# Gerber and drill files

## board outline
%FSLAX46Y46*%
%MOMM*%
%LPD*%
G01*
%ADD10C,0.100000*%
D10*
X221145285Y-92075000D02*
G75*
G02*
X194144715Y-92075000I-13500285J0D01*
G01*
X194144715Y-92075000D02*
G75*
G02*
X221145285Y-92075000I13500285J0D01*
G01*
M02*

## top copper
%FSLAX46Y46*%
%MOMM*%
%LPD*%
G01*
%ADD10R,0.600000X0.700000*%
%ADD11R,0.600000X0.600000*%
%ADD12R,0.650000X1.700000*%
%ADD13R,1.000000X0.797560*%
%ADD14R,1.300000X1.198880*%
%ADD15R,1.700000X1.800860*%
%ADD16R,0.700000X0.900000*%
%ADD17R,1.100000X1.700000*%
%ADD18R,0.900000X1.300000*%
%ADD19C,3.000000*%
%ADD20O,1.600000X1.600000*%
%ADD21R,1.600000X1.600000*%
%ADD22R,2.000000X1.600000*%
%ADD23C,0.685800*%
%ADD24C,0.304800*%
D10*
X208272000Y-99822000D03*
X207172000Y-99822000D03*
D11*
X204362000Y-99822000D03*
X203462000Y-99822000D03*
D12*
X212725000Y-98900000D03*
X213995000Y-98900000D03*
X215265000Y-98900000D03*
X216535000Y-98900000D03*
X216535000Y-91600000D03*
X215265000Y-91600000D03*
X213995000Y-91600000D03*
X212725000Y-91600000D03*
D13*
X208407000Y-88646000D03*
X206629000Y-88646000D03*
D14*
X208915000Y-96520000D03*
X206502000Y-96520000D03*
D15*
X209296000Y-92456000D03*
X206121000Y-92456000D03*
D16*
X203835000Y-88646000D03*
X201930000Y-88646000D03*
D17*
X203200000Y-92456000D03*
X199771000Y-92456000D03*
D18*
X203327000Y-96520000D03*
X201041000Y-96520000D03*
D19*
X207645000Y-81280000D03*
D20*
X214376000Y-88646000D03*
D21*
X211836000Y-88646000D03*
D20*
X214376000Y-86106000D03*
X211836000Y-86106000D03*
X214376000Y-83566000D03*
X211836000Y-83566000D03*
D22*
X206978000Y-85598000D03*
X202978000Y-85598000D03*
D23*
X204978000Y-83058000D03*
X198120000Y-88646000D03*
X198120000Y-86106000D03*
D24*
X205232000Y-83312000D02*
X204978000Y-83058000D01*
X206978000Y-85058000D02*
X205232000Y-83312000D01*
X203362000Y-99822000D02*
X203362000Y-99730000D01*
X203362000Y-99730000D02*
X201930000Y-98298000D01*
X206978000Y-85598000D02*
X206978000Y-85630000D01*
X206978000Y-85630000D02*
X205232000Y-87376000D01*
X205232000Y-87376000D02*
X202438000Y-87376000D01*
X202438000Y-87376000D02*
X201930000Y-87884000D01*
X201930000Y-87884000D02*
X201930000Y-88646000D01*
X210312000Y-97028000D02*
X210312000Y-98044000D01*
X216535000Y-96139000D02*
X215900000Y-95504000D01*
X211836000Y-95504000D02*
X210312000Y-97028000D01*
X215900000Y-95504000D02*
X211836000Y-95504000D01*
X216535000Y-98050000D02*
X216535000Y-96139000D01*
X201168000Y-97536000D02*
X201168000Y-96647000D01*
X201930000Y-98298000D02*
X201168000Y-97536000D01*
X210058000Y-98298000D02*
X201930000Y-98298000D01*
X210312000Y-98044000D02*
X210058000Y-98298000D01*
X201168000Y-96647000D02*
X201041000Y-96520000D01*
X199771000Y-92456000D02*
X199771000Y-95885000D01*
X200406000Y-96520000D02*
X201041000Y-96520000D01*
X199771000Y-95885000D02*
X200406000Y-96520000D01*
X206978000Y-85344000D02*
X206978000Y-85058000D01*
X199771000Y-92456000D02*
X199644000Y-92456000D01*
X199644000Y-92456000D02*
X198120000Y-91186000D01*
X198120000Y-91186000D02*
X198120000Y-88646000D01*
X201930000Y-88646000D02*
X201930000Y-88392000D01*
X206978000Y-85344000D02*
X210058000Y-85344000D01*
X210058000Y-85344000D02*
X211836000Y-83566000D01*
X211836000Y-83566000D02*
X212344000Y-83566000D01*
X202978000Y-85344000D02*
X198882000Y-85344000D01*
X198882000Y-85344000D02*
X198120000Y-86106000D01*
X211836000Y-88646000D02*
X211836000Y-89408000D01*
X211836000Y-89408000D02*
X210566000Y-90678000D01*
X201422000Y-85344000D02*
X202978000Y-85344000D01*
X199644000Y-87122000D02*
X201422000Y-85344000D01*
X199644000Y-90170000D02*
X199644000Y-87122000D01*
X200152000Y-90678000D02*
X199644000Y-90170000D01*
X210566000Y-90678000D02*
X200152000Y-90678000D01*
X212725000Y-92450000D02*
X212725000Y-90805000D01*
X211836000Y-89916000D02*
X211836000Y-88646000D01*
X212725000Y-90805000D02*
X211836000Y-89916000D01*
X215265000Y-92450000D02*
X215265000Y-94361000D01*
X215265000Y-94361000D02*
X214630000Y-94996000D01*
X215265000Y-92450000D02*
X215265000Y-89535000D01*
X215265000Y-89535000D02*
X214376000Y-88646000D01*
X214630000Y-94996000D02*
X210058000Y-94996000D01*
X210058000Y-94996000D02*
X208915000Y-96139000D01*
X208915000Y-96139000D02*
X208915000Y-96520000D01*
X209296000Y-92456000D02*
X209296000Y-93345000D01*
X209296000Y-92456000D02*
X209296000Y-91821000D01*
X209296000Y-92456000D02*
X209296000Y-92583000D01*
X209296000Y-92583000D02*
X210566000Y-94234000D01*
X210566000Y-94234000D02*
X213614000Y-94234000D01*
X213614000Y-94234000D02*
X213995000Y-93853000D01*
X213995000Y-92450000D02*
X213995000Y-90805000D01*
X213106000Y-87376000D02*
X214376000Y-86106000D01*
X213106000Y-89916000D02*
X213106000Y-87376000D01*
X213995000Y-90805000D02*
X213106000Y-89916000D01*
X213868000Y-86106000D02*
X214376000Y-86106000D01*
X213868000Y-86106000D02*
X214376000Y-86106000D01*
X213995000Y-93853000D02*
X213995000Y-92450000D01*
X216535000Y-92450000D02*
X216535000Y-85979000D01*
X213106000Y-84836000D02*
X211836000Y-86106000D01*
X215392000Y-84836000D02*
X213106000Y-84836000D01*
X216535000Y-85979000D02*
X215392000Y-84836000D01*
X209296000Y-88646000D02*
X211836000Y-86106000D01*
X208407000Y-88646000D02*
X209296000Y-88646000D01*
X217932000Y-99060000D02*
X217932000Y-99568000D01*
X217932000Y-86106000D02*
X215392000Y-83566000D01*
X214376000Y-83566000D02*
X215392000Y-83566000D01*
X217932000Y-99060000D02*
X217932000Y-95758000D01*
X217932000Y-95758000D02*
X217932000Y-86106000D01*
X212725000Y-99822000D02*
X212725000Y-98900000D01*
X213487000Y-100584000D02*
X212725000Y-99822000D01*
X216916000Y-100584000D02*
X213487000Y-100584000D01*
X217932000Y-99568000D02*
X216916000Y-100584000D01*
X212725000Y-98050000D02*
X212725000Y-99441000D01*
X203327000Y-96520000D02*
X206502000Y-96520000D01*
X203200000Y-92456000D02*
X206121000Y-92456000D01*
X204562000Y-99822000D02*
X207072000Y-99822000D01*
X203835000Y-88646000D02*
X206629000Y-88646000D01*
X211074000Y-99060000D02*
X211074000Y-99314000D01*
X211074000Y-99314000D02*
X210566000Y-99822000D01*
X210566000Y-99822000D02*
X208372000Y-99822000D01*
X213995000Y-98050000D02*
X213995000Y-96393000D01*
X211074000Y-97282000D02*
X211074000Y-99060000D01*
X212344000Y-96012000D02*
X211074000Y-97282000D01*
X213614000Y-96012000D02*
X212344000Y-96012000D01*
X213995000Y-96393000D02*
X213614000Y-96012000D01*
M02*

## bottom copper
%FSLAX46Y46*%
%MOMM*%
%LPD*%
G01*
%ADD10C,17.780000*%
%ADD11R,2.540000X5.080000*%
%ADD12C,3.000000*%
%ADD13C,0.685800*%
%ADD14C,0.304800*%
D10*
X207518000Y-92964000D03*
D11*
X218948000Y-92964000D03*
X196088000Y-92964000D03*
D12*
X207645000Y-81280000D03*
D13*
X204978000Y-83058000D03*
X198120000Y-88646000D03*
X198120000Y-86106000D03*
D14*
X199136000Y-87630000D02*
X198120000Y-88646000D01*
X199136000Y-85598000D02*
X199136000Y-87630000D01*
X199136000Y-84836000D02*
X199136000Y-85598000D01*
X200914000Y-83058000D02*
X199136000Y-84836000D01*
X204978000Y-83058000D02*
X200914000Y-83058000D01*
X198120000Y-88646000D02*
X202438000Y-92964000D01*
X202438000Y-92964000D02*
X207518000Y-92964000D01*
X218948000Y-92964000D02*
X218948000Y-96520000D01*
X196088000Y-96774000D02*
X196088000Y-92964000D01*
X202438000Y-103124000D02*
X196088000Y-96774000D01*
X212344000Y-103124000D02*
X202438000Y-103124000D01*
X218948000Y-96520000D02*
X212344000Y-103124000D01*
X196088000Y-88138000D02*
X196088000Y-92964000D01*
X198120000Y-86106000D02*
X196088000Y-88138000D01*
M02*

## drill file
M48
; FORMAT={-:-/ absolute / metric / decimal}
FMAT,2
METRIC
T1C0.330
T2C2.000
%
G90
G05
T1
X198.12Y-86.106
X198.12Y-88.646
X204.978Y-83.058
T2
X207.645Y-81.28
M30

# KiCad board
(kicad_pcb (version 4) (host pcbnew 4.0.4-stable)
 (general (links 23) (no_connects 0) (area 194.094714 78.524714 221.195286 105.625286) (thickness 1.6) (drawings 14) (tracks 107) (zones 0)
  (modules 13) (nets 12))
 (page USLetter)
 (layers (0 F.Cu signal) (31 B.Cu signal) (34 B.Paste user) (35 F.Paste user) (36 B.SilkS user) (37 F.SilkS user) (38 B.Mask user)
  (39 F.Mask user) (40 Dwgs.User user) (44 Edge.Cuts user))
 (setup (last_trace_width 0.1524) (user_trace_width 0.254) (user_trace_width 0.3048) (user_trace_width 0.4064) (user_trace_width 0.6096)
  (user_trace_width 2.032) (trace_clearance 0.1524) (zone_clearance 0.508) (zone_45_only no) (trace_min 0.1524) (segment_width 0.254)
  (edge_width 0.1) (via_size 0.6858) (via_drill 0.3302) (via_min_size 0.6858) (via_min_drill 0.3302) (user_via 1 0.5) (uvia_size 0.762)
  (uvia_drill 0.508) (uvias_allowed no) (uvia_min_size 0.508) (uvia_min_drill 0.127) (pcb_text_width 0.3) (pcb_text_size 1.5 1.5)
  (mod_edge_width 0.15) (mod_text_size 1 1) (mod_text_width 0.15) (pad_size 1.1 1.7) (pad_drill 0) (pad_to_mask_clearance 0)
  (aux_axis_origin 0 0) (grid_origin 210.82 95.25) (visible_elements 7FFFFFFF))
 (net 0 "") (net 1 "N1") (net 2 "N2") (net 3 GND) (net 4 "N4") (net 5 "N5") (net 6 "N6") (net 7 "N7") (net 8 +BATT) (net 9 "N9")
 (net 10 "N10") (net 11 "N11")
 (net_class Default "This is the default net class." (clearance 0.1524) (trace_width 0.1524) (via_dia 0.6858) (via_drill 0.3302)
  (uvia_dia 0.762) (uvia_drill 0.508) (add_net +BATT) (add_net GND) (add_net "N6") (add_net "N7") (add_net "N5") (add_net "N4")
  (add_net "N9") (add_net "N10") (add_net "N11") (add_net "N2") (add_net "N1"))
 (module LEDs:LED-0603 (layer F.Cu) (at 207.772 99.822)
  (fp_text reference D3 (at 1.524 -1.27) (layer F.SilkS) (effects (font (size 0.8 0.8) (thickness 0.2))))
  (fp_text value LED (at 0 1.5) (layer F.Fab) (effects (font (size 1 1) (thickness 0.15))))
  (pad 2 smd rect (at 0.5 0 180) (size 0.6 0.7) (layers F.Cu F.Paste F.Mask) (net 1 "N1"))
  (pad 1 smd rect (at -0.6 0 180) (size 0.6 0.7) (layers F.Cu F.Paste F.Mask) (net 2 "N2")))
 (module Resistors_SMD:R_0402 (layer F.Cu) (at 203.962 99.822 180)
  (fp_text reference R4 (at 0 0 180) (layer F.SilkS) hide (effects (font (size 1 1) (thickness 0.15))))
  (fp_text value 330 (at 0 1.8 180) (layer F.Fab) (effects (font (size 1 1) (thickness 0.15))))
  (pad 1 smd rect (at -0.4 0 180) (size 0.6 0.6) (layers F.Cu F.Paste F.Mask) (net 2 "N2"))
  (pad 2 smd rect (at 0.5 0 180) (size 0.6 0.6) (layers F.Cu F.Paste F.Mask) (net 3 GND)))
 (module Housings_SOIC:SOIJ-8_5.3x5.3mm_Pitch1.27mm (layer F.Cu) (at 214.63 95.25 90)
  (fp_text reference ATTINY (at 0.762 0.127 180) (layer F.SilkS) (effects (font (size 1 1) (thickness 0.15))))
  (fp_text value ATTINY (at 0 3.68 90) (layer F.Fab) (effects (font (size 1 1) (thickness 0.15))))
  (pad 1 smd rect (at -3.65 -1.905 90) (size 1.7 0.65) (layers F.Cu F.Paste F.Mask) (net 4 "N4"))
  (pad 2 smd rect (at -3.65 -0.635 90) (size 1.7 0.65) (layers F.Cu F.Paste F.Mask) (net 1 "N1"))
  (pad 3 smd rect (at -3.65 0.635 90) (size 1.7 0.65) (layers F.Cu F.Paste F.Mask))
  (pad 4 smd rect (at -3.65 1.905 90) (size 1.7 0.65) (layers F.Cu F.Paste F.Mask) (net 3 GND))
  (pad 5 smd rect (at 3.65 1.905 90) (size 1.7 0.65) (layers F.Cu F.Paste F.Mask) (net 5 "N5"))
  (pad 6 smd rect (at 3.65 0.635 90) (size 1.7 0.65) (layers F.Cu F.Paste F.Mask) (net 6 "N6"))
  (pad 7 smd rect (at 3.65 -0.635 90) (size 1.7 0.65) (layers F.Cu F.Paste F.Mask) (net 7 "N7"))
  (pad 8 smd rect (at 3.65 -1.905 90) (size 1.7 0.65) (layers F.Cu F.Paste F.Mask) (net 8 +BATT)))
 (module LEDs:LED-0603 (layer F.Cu) (at 207.518 88.646)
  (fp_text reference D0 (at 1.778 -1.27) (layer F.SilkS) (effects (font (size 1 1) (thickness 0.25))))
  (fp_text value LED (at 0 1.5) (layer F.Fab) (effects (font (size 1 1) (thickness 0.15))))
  (pad 2 smd rect (at 0.889 0 180) (size 1 0.79756) (layers F.Cu F.Paste F.Mask) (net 5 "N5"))
  (pad 1 smd rect (at -0.889 0 180) (size 1 0.79756) (layers F.Cu F.Paste F.Mask) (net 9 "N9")))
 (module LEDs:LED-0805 (layer F.Cu) (at 207.772 96.52)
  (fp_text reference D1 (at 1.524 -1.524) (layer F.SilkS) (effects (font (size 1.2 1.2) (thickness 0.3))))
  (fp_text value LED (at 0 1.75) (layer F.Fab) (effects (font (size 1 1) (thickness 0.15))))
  (pad 2 smd rect (at 1.143 0 180) (size 1.3 1.19888) (layers F.Cu F.Paste F.Mask) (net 6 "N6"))
  (pad 1 smd rect (at -1.27 0 180) (size 1.3 1.19888) (layers F.Cu F.Paste F.Mask) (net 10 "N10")))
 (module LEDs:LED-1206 (layer F.Cu) (at 207.772 92.456)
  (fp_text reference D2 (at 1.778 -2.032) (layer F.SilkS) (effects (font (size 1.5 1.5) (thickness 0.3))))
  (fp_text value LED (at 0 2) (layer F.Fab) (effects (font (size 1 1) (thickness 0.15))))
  (pad 2 smd rect (at 1.524 0 180) (size 1.7 1.80086) (layers F.Cu F.Paste F.Mask) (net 7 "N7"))
  (pad 1 smd rect (at -1.651 0 180) (size 1.7 1.80086) (layers F.Cu F.Paste F.Mask) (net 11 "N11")))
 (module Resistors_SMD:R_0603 (layer F.Cu) (at 202.946 88.646 180)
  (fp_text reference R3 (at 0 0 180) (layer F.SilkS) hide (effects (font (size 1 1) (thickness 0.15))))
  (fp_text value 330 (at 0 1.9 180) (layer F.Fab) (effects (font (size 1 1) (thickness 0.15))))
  (pad 1 smd rect (at -0.889 0 180) (size 0.7 0.9) (layers F.Cu F.Paste F.Mask) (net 9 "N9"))
  (pad 2 smd rect (at 1.016 0 180) (size 0.7 0.9) (layers F.Cu F.Paste F.Mask) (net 3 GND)))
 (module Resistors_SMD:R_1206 (layer F.Cu) (at 201.422 92.456 180)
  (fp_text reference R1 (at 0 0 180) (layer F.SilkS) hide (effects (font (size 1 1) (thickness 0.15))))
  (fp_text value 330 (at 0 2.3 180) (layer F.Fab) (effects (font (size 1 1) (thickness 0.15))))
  (pad 1 smd rect (at -1.778 0 180) (size 1.1 1.7) (layers F.Cu F.Paste F.Mask) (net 11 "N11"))
  (pad 2 smd rect (at 1.651 0 180) (size 1.1 1.7) (layers F.Cu F.Paste F.Mask) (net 3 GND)))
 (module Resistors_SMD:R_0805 (layer F.Cu) (at 202.184 96.52 180)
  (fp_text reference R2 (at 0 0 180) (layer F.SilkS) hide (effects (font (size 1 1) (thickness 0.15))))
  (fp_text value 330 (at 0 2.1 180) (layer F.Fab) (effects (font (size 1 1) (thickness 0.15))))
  (pad 1 smd rect (at -1.143 0 180) (size 0.9 1.3) (layers F.Cu F.Paste F.Mask) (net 10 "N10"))
  (pad 2 smd rect (at 1.143 0 180) (size 0.9 1.3) (layers F.Cu F.Paste F.Mask) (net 3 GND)))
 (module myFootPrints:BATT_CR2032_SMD (layer B.Cu) (at 207.518 92.964 180)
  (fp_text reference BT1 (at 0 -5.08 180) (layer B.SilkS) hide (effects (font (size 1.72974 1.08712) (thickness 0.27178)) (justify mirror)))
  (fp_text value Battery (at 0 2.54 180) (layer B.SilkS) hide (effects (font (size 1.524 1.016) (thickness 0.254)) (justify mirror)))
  (pad 2 smd circle (at 0 0 180) (size 17.78 17.78) (layers B.Cu B.Paste B.Mask) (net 3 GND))
  (pad 1 smd rect (at -11.43 0 180) (size 2.54 5.08) (layers B.Cu B.Paste B.Mask) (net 8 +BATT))
  (pad 1 smd rect (at 11.43 0 180) (size 2.54 5.08) (layers B.Cu B.Paste B.Mask) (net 8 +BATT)))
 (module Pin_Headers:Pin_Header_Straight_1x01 (layer F.Cu) (at 207.645 81.28)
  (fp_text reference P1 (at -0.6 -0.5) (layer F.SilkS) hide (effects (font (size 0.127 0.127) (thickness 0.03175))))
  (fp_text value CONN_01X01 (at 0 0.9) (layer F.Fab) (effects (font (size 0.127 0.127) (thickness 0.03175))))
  (pad "" thru_hole circle (at 0 0) (size 3 3) (drill 2) (layers *.Cu *.Mask)))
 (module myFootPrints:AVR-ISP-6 (layer F.Cu) (at 214.376 88.646 180)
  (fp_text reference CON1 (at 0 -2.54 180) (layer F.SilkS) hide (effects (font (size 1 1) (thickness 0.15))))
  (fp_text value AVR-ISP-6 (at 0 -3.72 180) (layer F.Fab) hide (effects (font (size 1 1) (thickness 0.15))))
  (pad 1 smd oval (at 0 0 180) (size 1.6 1.6) (layers F.Cu F.Paste F.Mask) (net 6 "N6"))
  (pad 2 smd rect (at 2.54 0 180) (size 1.6 1.6) (layers F.Cu F.Paste F.Mask) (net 8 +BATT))
  (pad 3 smd oval (at 0 2.54 180) (size 1.6 1.6) (layers F.Cu F.Paste F.Mask) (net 7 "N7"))
  (pad 4 smd oval (at 2.54 2.54 180) (size 1.6 1.6) (layers F.Cu F.Paste F.Mask) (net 5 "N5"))
  (pad 5 smd oval (at 0 5.08 180) (size 1.6 1.6) (layers F.Cu F.Paste F.Mask) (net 4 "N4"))
  (pad 6 smd oval (at 2.54 5.08 180) (size 1.6 1.6) (layers F.Cu F.Paste F.Mask) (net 3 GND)))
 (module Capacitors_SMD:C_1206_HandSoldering (layer F.Cu) (at 204.978 85.598 180)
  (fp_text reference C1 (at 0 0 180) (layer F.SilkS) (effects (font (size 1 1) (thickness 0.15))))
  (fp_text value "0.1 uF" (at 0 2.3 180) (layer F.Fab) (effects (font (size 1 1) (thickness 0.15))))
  (pad 1 smd rect (at -2 0 180) (size 2 1.6) (layers F.Cu F.Paste F.Mask) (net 3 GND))
  (pad 2 smd rect (at 2 0 180) (size 2 1.6) (layers F.Cu F.Paste F.Mask) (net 8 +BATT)))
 (gr_circle (center 207.645 92.075) (end 197.485 83.185) (layer Edge.Cuts) (width 0.1))
 (segment (start 205.232 83.312) (end 204.978 83.058) (width 0.3048) (layer F.Cu) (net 3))
 (segment (start 206.978 85.058) (end 205.232 83.312) (width 0.3048) (layer F.Cu) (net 3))
 (segment (start 199.136 87.63) (end 198.12 88.646) (width 0.3048) (layer B.Cu) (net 3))
 (segment (start 199.136 85.598) (end 199.136 87.63) (width 0.3048) (layer B.Cu) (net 3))
 (segment (start 199.136 84.836) (end 199.136 85.598) (width 0.3048) (layer B.Cu) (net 3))
 (segment (start 200.914 83.058) (end 199.136 84.836) (width 0.3048) (layer B.Cu) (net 3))
 (segment (start 204.978 83.058) (end 200.914 83.058) (width 0.3048) (layer B.Cu) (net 3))
 (via (at 204.978 83.058) (size 0.6858) (drill 0.3302) (layers F.Cu B.Cu) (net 3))
 (segment (start 203.362 99.822) (end 203.362 99.73) (width 0.3048) (layer F.Cu) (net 3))
 (segment (start 203.362 99.73) (end 201.93 98.298) (width 0.3048) (layer F.Cu) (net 3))
 (segment (start 206.978 85.598) (end 206.978 85.63) (width 0.3048) (layer F.Cu) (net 3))
 (segment (start 206.978 85.63) (end 205.232 87.376) (width 0.3048) (layer F.Cu) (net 3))
 (segment (start 205.232 87.376) (end 202.438 87.376) (width 0.3048) (layer F.Cu) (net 3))
 (segment (start 202.438 87.376) (end 201.93 87.884) (width 0.3048) (layer F.Cu) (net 3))
 (segment (start 201.93 87.884) (end 201.93 88.646) (width 0.3048) (layer F.Cu) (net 3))
 (segment (start 210.312 97.028) (end 210.312 98.044) (width 0.3048) (layer F.Cu) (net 3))
 (segment (start 216.535 96.139) (end 215.9 95.504) (width 0.3048) (layer F.Cu) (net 3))
 (segment (start 211.836 95.504) (end 210.312 97.028) (width 0.3048) (layer F.Cu) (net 3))
 (segment (start 215.9 95.504) (end 211.836 95.504) (width 0.3048) (layer F.Cu) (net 3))
 (segment (start 216.535 98.05) (end 216.535 96.139) (width 0.3048) (layer F.Cu) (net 3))
 (segment (start 201.168 97.536) (end 201.168 96.647) (width 0.3048) (layer F.Cu) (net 3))
 (segment (start 201.93 98.298) (end 201.168 97.536) (width 0.3048) (layer F.Cu) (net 3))
 (segment (start 210.058 98.298) (end 201.93 98.298) (width 0.3048) (layer F.Cu) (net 3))
 (segment (start 210.312 98.044) (end 210.058 98.298) (width 0.3048) (layer F.Cu) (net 3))
 (segment (start 201.168 96.647) (end 201.041 96.52) (width 0.3048) (layer F.Cu) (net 3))
 (segment (start 199.771 92.456) (end 199.771 95.885) (width 0.3048) (layer F.Cu) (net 3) (status 10))
 (segment (start 200.406 96.52) (end 201.041 96.52) (width 0.3048) (layer F.Cu) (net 3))
 (segment (start 199.771 95.885) (end 200.406 96.52) (width 0.3048) (layer F.Cu) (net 3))
 (segment (start 206.978 85.344) (end 206.978 85.058) (width 0.3048) (layer F.Cu) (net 3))
 (segment (start 199.771 92.456) (end 199.644 92.456) (width 0.3048) (layer F.Cu) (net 3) (status 30))
 (segment (start 198.12 88.646) (end 202.438 92.964) (width 0.3048) (layer B.Cu) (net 3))
 (via (at 198.12 88.646) (size 0.6858) (drill 0.3302) (layers F.Cu B.Cu) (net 3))
 (segment (start 199.644 92.456) (end 198.12 91.186) (width 0.3048) (layer F.Cu) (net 3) (status 10))
 (segment (start 198.12 91.186) (end 198.12 88.646) (width 0.3048) (layer F.Cu) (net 3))
 (segment (start 202.438 92.964) (end 207.518 92.964) (width 0.3048) (layer B.Cu) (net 3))
 (segment (start 201.93 88.646) (end 201.93 88.392) (width 0.3048) (layer F.Cu) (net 3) (status 30))
 (segment (start 206.978 85.344) (end 210.058 85.344) (width 0.3048) (layer F.Cu) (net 3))
 (segment (start 210.058 85.344) (end 211.836 83.566) (width 0.3048) (layer F.Cu) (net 3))
 (segment (start 211.836 83.566) (end 212.344 83.566) (width 0.3048) (layer F.Cu) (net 3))
 (segment (start 218.948 92.964) (end 218.948 96.52) (width 0.3048) (layer B.Cu) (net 8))
 (segment (start 196.088 96.774) (end 196.088 92.964) (width 0.3048) (layer B.Cu) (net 8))
 (segment (start 202.438 103.124) (end 196.088 96.774) (width 0.3048) (layer B.Cu) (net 8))
 (segment (start 212.344 103.124) (end 202.438 103.124) (width 0.3048) (layer B.Cu) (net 8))
 (segment (start 218.948 96.52) (end 212.344 103.124) (width 0.3048) (layer B.Cu) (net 8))
 (segment (start 202.978 85.344) (end 198.882 85.344) (width 0.3048) (layer F.Cu) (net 8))
 (segment (start 196.088 88.138) (end 196.088 92.964) (width 0.3048) (layer B.Cu) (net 8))
 (segment (start 198.12 86.106) (end 196.088 88.138) (width 0.3048) (layer B.Cu) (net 8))
 (via (at 198.12 86.106) (size 0.6858) (drill 0.3302) (layers F.Cu B.Cu) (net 8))
 (segment (start 198.882 85.344) (end 198.12 86.106) (width 0.3048) (layer F.Cu) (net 8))
 (segment (start 211.836 88.646) (end 211.836 89.408) (width 0.3048) (layer F.Cu) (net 8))
 (segment (start 211.836 89.408) (end 210.566 90.678) (width 0.3048) (layer F.Cu) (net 8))
 (segment (start 201.422 85.344) (end 202.978 85.344) (width 0.3048) (layer F.Cu) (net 8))
 (segment (start 199.644 87.122) (end 201.422 85.344) (width 0.3048) (layer F.Cu) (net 8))
 (segment (start 199.644 90.17) (end 199.644 87.122) (width 0.3048) (layer F.Cu) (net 8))
 (segment (start 200.152 90.678) (end 199.644 90.17) (width 0.3048) (layer F.Cu) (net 8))
 (segment (start 210.566 90.678) (end 200.152 90.678) (width 0.3048) (layer F.Cu) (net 8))
 (segment (start 212.725 92.45) (end 212.725 90.805) (width 0.3048) (layer F.Cu) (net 8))
 (segment (start 211.836 89.916) (end 211.836 88.646) (width 0.3048) (layer F.Cu) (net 8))
 (segment (start 212.725 90.805) (end 211.836 89.916) (width 0.3048) (layer F.Cu) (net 8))
 (segment (start 215.265 92.45) (end 215.265 94.361) (width 0.3048) (layer F.Cu) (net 6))
 (segment (start 215.265 94.361) (end 214.63 94.996) (width 0.3048) (layer F.Cu) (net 6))
 (segment (start 215.265 92.45) (end 215.265 89.535) (width 0.3048) (layer F.Cu) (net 6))
 (segment (start 215.265 89.535) (end 214.376 88.646) (width 0.3048) (layer F.Cu) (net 6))
 (segment (start 214.63 94.996) (end 210.058 94.996) (width 0.3048) (layer F.Cu) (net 6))
 (segment (start 210.058 94.996) (end 208.915 96.139) (width 0.3048) (layer F.Cu) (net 6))
 (segment (start 208.915 96.139) (end 208.915 96.52) (width 0.3048) (layer F.Cu) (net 6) (status 20))
 (segment (start 209.296 92.456) (end 209.296 93.345) (width 0.3048) (layer F.Cu) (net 7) (status 30))
 (segment (start 209.296 92.456) (end 209.296 91.821) (width 0.3048) (layer F.Cu) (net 7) (status 30))
 (segment (start 209.296 92.456) (end 209.296 92.583) (width 0.3048) (layer F.Cu) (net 7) (status 30))
 (segment (start 209.296 92.583) (end 210.566 94.234) (width 0.3048) (layer F.Cu) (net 7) (status 10))
 (segment (start 210.566 94.234) (end 213.614 94.234) (width 0.3048) (layer F.Cu) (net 7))
 (segment (start 213.614 94.234) (end 213.995 93.853) (width 0.3048) (layer F.Cu) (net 7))
 (segment (start 213.995 92.45) (end 213.995 90.805) (width 0.3048) (layer F.Cu) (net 7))
 (segment (start 213.106 87.376) (end 214.376 86.106) (width 0.3048) (layer F.Cu) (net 7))
 (segment (start 213.106 89.916) (end 213.106 87.376) (width 0.3048) (layer F.Cu) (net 7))
 (segment (start 213.995 90.805) (end 213.106 89.916) (width 0.3048) (layer F.Cu) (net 7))
 (segment (start 213.868 86.106) (end 214.376 86.106) (width 0.3048) (layer F.Cu) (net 7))
 (segment (start 213.868 86.106) (end 214.376 86.106) (width 0.3048) (layer F.Cu) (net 7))
 (segment (start 213.995 93.853) (end 213.995 92.45) (width 0.3048) (layer F.Cu) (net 7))
 (segment (start 216.535 92.45) (end 216.535 85.979) (width 0.3048) (layer F.Cu) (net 5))
 (segment (start 213.106 84.836) (end 211.836 86.106) (width 0.3048) (layer F.Cu) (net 5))
 (segment (start 215.392 84.836) (end 213.106 84.836) (width 0.3048) (layer F.Cu) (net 5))
 (segment (start 216.535 85.979) (end 215.392 84.836) (width 0.3048) (layer F.Cu) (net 5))
 (segment (start 209.296 88.646) (end 211.836 86.106) (width 0.3048) (layer F.Cu) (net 5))
 (segment (start 208.407 88.646) (end 209.296 88.646) (width 0.3048) (layer F.Cu) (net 5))
 (segment (start 217.932 99.06) (end 217.932 99.568) (width 0.3048) (layer F.Cu) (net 4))
 (segment (start 217.932 86.106) (end 215.392 83.566) (width 0.3048) (layer F.Cu) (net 4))
 (segment (start 214.376 83.566) (end 215.392 83.566) (width 0.3048) (layer F.Cu) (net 4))
 (segment (start 217.932 99.06) (end 217.932 95.758) (width 0.3048) (layer F.Cu) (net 4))
 (segment (start 217.932 95.758) (end 217.932 86.106) (width 0.3048) (layer F.Cu) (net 4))
 (segment (start 212.725 99.822) (end 212.725 98.9) (width 0.3048) (layer F.Cu) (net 4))
 (segment (start 213.487 100.584) (end 212.725 99.822) (width 0.3048) (layer F.Cu) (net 4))
 (segment (start 216.916 100.584) (end 213.487 100.584) (width 0.3048) (layer F.Cu) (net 4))
 (segment (start 217.932 99.568) (end 216.916 100.584) (width 0.3048) (layer F.Cu) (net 4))
 (segment (start 212.725 98.05) (end 212.725 99.441) (width 0.3048) (layer F.Cu) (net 4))
 (segment (start 203.327 96.52) (end 206.502 96.52) (width 0.3048) (layer F.Cu) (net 10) (status 10))
 (segment (start 203.2 92.456) (end 206.121 92.456) (width 0.3048) (layer F.Cu) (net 11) (status 10))
 (segment (start 204.562 99.822) (end 207.072 99.822) (width 0.3048) (layer F.Cu) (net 2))
 (segment (start 203.835 88.646) (end 206.629 88.646) (width 0.3048) (layer F.Cu) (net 9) (status 10))
 (segment (start 211.074 99.06) (end 211.074 99.314) (width 0.3048) (layer F.Cu) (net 1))
 (segment (start 211.074 99.314) (end 210.566 99.822) (width 0.3048) (layer F.Cu) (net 1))
 (segment (start 210.566 99.822) (end 208.372 99.822) (width 0.3048) (layer F.Cu) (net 1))
 (segment (start 213.995 98.05) (end 213.995 96.393) (width 0.3048) (layer F.Cu) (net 1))
 (segment (start 211.074 97.282) (end 211.074 99.06) (width 0.3048) (layer F.Cu) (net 1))
 (segment (start 212.344 96.012) (end 211.074 97.282) (width 0.3048) (layer F.Cu) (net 1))
 (segment (start 213.614 96.012) (end 212.344 96.012) (width 0.3048) (layer F.Cu) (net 1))
 (segment (start 213.995 96.393) (end 213.614 96.012) (width 0.3048) (layer F.Cu) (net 1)))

